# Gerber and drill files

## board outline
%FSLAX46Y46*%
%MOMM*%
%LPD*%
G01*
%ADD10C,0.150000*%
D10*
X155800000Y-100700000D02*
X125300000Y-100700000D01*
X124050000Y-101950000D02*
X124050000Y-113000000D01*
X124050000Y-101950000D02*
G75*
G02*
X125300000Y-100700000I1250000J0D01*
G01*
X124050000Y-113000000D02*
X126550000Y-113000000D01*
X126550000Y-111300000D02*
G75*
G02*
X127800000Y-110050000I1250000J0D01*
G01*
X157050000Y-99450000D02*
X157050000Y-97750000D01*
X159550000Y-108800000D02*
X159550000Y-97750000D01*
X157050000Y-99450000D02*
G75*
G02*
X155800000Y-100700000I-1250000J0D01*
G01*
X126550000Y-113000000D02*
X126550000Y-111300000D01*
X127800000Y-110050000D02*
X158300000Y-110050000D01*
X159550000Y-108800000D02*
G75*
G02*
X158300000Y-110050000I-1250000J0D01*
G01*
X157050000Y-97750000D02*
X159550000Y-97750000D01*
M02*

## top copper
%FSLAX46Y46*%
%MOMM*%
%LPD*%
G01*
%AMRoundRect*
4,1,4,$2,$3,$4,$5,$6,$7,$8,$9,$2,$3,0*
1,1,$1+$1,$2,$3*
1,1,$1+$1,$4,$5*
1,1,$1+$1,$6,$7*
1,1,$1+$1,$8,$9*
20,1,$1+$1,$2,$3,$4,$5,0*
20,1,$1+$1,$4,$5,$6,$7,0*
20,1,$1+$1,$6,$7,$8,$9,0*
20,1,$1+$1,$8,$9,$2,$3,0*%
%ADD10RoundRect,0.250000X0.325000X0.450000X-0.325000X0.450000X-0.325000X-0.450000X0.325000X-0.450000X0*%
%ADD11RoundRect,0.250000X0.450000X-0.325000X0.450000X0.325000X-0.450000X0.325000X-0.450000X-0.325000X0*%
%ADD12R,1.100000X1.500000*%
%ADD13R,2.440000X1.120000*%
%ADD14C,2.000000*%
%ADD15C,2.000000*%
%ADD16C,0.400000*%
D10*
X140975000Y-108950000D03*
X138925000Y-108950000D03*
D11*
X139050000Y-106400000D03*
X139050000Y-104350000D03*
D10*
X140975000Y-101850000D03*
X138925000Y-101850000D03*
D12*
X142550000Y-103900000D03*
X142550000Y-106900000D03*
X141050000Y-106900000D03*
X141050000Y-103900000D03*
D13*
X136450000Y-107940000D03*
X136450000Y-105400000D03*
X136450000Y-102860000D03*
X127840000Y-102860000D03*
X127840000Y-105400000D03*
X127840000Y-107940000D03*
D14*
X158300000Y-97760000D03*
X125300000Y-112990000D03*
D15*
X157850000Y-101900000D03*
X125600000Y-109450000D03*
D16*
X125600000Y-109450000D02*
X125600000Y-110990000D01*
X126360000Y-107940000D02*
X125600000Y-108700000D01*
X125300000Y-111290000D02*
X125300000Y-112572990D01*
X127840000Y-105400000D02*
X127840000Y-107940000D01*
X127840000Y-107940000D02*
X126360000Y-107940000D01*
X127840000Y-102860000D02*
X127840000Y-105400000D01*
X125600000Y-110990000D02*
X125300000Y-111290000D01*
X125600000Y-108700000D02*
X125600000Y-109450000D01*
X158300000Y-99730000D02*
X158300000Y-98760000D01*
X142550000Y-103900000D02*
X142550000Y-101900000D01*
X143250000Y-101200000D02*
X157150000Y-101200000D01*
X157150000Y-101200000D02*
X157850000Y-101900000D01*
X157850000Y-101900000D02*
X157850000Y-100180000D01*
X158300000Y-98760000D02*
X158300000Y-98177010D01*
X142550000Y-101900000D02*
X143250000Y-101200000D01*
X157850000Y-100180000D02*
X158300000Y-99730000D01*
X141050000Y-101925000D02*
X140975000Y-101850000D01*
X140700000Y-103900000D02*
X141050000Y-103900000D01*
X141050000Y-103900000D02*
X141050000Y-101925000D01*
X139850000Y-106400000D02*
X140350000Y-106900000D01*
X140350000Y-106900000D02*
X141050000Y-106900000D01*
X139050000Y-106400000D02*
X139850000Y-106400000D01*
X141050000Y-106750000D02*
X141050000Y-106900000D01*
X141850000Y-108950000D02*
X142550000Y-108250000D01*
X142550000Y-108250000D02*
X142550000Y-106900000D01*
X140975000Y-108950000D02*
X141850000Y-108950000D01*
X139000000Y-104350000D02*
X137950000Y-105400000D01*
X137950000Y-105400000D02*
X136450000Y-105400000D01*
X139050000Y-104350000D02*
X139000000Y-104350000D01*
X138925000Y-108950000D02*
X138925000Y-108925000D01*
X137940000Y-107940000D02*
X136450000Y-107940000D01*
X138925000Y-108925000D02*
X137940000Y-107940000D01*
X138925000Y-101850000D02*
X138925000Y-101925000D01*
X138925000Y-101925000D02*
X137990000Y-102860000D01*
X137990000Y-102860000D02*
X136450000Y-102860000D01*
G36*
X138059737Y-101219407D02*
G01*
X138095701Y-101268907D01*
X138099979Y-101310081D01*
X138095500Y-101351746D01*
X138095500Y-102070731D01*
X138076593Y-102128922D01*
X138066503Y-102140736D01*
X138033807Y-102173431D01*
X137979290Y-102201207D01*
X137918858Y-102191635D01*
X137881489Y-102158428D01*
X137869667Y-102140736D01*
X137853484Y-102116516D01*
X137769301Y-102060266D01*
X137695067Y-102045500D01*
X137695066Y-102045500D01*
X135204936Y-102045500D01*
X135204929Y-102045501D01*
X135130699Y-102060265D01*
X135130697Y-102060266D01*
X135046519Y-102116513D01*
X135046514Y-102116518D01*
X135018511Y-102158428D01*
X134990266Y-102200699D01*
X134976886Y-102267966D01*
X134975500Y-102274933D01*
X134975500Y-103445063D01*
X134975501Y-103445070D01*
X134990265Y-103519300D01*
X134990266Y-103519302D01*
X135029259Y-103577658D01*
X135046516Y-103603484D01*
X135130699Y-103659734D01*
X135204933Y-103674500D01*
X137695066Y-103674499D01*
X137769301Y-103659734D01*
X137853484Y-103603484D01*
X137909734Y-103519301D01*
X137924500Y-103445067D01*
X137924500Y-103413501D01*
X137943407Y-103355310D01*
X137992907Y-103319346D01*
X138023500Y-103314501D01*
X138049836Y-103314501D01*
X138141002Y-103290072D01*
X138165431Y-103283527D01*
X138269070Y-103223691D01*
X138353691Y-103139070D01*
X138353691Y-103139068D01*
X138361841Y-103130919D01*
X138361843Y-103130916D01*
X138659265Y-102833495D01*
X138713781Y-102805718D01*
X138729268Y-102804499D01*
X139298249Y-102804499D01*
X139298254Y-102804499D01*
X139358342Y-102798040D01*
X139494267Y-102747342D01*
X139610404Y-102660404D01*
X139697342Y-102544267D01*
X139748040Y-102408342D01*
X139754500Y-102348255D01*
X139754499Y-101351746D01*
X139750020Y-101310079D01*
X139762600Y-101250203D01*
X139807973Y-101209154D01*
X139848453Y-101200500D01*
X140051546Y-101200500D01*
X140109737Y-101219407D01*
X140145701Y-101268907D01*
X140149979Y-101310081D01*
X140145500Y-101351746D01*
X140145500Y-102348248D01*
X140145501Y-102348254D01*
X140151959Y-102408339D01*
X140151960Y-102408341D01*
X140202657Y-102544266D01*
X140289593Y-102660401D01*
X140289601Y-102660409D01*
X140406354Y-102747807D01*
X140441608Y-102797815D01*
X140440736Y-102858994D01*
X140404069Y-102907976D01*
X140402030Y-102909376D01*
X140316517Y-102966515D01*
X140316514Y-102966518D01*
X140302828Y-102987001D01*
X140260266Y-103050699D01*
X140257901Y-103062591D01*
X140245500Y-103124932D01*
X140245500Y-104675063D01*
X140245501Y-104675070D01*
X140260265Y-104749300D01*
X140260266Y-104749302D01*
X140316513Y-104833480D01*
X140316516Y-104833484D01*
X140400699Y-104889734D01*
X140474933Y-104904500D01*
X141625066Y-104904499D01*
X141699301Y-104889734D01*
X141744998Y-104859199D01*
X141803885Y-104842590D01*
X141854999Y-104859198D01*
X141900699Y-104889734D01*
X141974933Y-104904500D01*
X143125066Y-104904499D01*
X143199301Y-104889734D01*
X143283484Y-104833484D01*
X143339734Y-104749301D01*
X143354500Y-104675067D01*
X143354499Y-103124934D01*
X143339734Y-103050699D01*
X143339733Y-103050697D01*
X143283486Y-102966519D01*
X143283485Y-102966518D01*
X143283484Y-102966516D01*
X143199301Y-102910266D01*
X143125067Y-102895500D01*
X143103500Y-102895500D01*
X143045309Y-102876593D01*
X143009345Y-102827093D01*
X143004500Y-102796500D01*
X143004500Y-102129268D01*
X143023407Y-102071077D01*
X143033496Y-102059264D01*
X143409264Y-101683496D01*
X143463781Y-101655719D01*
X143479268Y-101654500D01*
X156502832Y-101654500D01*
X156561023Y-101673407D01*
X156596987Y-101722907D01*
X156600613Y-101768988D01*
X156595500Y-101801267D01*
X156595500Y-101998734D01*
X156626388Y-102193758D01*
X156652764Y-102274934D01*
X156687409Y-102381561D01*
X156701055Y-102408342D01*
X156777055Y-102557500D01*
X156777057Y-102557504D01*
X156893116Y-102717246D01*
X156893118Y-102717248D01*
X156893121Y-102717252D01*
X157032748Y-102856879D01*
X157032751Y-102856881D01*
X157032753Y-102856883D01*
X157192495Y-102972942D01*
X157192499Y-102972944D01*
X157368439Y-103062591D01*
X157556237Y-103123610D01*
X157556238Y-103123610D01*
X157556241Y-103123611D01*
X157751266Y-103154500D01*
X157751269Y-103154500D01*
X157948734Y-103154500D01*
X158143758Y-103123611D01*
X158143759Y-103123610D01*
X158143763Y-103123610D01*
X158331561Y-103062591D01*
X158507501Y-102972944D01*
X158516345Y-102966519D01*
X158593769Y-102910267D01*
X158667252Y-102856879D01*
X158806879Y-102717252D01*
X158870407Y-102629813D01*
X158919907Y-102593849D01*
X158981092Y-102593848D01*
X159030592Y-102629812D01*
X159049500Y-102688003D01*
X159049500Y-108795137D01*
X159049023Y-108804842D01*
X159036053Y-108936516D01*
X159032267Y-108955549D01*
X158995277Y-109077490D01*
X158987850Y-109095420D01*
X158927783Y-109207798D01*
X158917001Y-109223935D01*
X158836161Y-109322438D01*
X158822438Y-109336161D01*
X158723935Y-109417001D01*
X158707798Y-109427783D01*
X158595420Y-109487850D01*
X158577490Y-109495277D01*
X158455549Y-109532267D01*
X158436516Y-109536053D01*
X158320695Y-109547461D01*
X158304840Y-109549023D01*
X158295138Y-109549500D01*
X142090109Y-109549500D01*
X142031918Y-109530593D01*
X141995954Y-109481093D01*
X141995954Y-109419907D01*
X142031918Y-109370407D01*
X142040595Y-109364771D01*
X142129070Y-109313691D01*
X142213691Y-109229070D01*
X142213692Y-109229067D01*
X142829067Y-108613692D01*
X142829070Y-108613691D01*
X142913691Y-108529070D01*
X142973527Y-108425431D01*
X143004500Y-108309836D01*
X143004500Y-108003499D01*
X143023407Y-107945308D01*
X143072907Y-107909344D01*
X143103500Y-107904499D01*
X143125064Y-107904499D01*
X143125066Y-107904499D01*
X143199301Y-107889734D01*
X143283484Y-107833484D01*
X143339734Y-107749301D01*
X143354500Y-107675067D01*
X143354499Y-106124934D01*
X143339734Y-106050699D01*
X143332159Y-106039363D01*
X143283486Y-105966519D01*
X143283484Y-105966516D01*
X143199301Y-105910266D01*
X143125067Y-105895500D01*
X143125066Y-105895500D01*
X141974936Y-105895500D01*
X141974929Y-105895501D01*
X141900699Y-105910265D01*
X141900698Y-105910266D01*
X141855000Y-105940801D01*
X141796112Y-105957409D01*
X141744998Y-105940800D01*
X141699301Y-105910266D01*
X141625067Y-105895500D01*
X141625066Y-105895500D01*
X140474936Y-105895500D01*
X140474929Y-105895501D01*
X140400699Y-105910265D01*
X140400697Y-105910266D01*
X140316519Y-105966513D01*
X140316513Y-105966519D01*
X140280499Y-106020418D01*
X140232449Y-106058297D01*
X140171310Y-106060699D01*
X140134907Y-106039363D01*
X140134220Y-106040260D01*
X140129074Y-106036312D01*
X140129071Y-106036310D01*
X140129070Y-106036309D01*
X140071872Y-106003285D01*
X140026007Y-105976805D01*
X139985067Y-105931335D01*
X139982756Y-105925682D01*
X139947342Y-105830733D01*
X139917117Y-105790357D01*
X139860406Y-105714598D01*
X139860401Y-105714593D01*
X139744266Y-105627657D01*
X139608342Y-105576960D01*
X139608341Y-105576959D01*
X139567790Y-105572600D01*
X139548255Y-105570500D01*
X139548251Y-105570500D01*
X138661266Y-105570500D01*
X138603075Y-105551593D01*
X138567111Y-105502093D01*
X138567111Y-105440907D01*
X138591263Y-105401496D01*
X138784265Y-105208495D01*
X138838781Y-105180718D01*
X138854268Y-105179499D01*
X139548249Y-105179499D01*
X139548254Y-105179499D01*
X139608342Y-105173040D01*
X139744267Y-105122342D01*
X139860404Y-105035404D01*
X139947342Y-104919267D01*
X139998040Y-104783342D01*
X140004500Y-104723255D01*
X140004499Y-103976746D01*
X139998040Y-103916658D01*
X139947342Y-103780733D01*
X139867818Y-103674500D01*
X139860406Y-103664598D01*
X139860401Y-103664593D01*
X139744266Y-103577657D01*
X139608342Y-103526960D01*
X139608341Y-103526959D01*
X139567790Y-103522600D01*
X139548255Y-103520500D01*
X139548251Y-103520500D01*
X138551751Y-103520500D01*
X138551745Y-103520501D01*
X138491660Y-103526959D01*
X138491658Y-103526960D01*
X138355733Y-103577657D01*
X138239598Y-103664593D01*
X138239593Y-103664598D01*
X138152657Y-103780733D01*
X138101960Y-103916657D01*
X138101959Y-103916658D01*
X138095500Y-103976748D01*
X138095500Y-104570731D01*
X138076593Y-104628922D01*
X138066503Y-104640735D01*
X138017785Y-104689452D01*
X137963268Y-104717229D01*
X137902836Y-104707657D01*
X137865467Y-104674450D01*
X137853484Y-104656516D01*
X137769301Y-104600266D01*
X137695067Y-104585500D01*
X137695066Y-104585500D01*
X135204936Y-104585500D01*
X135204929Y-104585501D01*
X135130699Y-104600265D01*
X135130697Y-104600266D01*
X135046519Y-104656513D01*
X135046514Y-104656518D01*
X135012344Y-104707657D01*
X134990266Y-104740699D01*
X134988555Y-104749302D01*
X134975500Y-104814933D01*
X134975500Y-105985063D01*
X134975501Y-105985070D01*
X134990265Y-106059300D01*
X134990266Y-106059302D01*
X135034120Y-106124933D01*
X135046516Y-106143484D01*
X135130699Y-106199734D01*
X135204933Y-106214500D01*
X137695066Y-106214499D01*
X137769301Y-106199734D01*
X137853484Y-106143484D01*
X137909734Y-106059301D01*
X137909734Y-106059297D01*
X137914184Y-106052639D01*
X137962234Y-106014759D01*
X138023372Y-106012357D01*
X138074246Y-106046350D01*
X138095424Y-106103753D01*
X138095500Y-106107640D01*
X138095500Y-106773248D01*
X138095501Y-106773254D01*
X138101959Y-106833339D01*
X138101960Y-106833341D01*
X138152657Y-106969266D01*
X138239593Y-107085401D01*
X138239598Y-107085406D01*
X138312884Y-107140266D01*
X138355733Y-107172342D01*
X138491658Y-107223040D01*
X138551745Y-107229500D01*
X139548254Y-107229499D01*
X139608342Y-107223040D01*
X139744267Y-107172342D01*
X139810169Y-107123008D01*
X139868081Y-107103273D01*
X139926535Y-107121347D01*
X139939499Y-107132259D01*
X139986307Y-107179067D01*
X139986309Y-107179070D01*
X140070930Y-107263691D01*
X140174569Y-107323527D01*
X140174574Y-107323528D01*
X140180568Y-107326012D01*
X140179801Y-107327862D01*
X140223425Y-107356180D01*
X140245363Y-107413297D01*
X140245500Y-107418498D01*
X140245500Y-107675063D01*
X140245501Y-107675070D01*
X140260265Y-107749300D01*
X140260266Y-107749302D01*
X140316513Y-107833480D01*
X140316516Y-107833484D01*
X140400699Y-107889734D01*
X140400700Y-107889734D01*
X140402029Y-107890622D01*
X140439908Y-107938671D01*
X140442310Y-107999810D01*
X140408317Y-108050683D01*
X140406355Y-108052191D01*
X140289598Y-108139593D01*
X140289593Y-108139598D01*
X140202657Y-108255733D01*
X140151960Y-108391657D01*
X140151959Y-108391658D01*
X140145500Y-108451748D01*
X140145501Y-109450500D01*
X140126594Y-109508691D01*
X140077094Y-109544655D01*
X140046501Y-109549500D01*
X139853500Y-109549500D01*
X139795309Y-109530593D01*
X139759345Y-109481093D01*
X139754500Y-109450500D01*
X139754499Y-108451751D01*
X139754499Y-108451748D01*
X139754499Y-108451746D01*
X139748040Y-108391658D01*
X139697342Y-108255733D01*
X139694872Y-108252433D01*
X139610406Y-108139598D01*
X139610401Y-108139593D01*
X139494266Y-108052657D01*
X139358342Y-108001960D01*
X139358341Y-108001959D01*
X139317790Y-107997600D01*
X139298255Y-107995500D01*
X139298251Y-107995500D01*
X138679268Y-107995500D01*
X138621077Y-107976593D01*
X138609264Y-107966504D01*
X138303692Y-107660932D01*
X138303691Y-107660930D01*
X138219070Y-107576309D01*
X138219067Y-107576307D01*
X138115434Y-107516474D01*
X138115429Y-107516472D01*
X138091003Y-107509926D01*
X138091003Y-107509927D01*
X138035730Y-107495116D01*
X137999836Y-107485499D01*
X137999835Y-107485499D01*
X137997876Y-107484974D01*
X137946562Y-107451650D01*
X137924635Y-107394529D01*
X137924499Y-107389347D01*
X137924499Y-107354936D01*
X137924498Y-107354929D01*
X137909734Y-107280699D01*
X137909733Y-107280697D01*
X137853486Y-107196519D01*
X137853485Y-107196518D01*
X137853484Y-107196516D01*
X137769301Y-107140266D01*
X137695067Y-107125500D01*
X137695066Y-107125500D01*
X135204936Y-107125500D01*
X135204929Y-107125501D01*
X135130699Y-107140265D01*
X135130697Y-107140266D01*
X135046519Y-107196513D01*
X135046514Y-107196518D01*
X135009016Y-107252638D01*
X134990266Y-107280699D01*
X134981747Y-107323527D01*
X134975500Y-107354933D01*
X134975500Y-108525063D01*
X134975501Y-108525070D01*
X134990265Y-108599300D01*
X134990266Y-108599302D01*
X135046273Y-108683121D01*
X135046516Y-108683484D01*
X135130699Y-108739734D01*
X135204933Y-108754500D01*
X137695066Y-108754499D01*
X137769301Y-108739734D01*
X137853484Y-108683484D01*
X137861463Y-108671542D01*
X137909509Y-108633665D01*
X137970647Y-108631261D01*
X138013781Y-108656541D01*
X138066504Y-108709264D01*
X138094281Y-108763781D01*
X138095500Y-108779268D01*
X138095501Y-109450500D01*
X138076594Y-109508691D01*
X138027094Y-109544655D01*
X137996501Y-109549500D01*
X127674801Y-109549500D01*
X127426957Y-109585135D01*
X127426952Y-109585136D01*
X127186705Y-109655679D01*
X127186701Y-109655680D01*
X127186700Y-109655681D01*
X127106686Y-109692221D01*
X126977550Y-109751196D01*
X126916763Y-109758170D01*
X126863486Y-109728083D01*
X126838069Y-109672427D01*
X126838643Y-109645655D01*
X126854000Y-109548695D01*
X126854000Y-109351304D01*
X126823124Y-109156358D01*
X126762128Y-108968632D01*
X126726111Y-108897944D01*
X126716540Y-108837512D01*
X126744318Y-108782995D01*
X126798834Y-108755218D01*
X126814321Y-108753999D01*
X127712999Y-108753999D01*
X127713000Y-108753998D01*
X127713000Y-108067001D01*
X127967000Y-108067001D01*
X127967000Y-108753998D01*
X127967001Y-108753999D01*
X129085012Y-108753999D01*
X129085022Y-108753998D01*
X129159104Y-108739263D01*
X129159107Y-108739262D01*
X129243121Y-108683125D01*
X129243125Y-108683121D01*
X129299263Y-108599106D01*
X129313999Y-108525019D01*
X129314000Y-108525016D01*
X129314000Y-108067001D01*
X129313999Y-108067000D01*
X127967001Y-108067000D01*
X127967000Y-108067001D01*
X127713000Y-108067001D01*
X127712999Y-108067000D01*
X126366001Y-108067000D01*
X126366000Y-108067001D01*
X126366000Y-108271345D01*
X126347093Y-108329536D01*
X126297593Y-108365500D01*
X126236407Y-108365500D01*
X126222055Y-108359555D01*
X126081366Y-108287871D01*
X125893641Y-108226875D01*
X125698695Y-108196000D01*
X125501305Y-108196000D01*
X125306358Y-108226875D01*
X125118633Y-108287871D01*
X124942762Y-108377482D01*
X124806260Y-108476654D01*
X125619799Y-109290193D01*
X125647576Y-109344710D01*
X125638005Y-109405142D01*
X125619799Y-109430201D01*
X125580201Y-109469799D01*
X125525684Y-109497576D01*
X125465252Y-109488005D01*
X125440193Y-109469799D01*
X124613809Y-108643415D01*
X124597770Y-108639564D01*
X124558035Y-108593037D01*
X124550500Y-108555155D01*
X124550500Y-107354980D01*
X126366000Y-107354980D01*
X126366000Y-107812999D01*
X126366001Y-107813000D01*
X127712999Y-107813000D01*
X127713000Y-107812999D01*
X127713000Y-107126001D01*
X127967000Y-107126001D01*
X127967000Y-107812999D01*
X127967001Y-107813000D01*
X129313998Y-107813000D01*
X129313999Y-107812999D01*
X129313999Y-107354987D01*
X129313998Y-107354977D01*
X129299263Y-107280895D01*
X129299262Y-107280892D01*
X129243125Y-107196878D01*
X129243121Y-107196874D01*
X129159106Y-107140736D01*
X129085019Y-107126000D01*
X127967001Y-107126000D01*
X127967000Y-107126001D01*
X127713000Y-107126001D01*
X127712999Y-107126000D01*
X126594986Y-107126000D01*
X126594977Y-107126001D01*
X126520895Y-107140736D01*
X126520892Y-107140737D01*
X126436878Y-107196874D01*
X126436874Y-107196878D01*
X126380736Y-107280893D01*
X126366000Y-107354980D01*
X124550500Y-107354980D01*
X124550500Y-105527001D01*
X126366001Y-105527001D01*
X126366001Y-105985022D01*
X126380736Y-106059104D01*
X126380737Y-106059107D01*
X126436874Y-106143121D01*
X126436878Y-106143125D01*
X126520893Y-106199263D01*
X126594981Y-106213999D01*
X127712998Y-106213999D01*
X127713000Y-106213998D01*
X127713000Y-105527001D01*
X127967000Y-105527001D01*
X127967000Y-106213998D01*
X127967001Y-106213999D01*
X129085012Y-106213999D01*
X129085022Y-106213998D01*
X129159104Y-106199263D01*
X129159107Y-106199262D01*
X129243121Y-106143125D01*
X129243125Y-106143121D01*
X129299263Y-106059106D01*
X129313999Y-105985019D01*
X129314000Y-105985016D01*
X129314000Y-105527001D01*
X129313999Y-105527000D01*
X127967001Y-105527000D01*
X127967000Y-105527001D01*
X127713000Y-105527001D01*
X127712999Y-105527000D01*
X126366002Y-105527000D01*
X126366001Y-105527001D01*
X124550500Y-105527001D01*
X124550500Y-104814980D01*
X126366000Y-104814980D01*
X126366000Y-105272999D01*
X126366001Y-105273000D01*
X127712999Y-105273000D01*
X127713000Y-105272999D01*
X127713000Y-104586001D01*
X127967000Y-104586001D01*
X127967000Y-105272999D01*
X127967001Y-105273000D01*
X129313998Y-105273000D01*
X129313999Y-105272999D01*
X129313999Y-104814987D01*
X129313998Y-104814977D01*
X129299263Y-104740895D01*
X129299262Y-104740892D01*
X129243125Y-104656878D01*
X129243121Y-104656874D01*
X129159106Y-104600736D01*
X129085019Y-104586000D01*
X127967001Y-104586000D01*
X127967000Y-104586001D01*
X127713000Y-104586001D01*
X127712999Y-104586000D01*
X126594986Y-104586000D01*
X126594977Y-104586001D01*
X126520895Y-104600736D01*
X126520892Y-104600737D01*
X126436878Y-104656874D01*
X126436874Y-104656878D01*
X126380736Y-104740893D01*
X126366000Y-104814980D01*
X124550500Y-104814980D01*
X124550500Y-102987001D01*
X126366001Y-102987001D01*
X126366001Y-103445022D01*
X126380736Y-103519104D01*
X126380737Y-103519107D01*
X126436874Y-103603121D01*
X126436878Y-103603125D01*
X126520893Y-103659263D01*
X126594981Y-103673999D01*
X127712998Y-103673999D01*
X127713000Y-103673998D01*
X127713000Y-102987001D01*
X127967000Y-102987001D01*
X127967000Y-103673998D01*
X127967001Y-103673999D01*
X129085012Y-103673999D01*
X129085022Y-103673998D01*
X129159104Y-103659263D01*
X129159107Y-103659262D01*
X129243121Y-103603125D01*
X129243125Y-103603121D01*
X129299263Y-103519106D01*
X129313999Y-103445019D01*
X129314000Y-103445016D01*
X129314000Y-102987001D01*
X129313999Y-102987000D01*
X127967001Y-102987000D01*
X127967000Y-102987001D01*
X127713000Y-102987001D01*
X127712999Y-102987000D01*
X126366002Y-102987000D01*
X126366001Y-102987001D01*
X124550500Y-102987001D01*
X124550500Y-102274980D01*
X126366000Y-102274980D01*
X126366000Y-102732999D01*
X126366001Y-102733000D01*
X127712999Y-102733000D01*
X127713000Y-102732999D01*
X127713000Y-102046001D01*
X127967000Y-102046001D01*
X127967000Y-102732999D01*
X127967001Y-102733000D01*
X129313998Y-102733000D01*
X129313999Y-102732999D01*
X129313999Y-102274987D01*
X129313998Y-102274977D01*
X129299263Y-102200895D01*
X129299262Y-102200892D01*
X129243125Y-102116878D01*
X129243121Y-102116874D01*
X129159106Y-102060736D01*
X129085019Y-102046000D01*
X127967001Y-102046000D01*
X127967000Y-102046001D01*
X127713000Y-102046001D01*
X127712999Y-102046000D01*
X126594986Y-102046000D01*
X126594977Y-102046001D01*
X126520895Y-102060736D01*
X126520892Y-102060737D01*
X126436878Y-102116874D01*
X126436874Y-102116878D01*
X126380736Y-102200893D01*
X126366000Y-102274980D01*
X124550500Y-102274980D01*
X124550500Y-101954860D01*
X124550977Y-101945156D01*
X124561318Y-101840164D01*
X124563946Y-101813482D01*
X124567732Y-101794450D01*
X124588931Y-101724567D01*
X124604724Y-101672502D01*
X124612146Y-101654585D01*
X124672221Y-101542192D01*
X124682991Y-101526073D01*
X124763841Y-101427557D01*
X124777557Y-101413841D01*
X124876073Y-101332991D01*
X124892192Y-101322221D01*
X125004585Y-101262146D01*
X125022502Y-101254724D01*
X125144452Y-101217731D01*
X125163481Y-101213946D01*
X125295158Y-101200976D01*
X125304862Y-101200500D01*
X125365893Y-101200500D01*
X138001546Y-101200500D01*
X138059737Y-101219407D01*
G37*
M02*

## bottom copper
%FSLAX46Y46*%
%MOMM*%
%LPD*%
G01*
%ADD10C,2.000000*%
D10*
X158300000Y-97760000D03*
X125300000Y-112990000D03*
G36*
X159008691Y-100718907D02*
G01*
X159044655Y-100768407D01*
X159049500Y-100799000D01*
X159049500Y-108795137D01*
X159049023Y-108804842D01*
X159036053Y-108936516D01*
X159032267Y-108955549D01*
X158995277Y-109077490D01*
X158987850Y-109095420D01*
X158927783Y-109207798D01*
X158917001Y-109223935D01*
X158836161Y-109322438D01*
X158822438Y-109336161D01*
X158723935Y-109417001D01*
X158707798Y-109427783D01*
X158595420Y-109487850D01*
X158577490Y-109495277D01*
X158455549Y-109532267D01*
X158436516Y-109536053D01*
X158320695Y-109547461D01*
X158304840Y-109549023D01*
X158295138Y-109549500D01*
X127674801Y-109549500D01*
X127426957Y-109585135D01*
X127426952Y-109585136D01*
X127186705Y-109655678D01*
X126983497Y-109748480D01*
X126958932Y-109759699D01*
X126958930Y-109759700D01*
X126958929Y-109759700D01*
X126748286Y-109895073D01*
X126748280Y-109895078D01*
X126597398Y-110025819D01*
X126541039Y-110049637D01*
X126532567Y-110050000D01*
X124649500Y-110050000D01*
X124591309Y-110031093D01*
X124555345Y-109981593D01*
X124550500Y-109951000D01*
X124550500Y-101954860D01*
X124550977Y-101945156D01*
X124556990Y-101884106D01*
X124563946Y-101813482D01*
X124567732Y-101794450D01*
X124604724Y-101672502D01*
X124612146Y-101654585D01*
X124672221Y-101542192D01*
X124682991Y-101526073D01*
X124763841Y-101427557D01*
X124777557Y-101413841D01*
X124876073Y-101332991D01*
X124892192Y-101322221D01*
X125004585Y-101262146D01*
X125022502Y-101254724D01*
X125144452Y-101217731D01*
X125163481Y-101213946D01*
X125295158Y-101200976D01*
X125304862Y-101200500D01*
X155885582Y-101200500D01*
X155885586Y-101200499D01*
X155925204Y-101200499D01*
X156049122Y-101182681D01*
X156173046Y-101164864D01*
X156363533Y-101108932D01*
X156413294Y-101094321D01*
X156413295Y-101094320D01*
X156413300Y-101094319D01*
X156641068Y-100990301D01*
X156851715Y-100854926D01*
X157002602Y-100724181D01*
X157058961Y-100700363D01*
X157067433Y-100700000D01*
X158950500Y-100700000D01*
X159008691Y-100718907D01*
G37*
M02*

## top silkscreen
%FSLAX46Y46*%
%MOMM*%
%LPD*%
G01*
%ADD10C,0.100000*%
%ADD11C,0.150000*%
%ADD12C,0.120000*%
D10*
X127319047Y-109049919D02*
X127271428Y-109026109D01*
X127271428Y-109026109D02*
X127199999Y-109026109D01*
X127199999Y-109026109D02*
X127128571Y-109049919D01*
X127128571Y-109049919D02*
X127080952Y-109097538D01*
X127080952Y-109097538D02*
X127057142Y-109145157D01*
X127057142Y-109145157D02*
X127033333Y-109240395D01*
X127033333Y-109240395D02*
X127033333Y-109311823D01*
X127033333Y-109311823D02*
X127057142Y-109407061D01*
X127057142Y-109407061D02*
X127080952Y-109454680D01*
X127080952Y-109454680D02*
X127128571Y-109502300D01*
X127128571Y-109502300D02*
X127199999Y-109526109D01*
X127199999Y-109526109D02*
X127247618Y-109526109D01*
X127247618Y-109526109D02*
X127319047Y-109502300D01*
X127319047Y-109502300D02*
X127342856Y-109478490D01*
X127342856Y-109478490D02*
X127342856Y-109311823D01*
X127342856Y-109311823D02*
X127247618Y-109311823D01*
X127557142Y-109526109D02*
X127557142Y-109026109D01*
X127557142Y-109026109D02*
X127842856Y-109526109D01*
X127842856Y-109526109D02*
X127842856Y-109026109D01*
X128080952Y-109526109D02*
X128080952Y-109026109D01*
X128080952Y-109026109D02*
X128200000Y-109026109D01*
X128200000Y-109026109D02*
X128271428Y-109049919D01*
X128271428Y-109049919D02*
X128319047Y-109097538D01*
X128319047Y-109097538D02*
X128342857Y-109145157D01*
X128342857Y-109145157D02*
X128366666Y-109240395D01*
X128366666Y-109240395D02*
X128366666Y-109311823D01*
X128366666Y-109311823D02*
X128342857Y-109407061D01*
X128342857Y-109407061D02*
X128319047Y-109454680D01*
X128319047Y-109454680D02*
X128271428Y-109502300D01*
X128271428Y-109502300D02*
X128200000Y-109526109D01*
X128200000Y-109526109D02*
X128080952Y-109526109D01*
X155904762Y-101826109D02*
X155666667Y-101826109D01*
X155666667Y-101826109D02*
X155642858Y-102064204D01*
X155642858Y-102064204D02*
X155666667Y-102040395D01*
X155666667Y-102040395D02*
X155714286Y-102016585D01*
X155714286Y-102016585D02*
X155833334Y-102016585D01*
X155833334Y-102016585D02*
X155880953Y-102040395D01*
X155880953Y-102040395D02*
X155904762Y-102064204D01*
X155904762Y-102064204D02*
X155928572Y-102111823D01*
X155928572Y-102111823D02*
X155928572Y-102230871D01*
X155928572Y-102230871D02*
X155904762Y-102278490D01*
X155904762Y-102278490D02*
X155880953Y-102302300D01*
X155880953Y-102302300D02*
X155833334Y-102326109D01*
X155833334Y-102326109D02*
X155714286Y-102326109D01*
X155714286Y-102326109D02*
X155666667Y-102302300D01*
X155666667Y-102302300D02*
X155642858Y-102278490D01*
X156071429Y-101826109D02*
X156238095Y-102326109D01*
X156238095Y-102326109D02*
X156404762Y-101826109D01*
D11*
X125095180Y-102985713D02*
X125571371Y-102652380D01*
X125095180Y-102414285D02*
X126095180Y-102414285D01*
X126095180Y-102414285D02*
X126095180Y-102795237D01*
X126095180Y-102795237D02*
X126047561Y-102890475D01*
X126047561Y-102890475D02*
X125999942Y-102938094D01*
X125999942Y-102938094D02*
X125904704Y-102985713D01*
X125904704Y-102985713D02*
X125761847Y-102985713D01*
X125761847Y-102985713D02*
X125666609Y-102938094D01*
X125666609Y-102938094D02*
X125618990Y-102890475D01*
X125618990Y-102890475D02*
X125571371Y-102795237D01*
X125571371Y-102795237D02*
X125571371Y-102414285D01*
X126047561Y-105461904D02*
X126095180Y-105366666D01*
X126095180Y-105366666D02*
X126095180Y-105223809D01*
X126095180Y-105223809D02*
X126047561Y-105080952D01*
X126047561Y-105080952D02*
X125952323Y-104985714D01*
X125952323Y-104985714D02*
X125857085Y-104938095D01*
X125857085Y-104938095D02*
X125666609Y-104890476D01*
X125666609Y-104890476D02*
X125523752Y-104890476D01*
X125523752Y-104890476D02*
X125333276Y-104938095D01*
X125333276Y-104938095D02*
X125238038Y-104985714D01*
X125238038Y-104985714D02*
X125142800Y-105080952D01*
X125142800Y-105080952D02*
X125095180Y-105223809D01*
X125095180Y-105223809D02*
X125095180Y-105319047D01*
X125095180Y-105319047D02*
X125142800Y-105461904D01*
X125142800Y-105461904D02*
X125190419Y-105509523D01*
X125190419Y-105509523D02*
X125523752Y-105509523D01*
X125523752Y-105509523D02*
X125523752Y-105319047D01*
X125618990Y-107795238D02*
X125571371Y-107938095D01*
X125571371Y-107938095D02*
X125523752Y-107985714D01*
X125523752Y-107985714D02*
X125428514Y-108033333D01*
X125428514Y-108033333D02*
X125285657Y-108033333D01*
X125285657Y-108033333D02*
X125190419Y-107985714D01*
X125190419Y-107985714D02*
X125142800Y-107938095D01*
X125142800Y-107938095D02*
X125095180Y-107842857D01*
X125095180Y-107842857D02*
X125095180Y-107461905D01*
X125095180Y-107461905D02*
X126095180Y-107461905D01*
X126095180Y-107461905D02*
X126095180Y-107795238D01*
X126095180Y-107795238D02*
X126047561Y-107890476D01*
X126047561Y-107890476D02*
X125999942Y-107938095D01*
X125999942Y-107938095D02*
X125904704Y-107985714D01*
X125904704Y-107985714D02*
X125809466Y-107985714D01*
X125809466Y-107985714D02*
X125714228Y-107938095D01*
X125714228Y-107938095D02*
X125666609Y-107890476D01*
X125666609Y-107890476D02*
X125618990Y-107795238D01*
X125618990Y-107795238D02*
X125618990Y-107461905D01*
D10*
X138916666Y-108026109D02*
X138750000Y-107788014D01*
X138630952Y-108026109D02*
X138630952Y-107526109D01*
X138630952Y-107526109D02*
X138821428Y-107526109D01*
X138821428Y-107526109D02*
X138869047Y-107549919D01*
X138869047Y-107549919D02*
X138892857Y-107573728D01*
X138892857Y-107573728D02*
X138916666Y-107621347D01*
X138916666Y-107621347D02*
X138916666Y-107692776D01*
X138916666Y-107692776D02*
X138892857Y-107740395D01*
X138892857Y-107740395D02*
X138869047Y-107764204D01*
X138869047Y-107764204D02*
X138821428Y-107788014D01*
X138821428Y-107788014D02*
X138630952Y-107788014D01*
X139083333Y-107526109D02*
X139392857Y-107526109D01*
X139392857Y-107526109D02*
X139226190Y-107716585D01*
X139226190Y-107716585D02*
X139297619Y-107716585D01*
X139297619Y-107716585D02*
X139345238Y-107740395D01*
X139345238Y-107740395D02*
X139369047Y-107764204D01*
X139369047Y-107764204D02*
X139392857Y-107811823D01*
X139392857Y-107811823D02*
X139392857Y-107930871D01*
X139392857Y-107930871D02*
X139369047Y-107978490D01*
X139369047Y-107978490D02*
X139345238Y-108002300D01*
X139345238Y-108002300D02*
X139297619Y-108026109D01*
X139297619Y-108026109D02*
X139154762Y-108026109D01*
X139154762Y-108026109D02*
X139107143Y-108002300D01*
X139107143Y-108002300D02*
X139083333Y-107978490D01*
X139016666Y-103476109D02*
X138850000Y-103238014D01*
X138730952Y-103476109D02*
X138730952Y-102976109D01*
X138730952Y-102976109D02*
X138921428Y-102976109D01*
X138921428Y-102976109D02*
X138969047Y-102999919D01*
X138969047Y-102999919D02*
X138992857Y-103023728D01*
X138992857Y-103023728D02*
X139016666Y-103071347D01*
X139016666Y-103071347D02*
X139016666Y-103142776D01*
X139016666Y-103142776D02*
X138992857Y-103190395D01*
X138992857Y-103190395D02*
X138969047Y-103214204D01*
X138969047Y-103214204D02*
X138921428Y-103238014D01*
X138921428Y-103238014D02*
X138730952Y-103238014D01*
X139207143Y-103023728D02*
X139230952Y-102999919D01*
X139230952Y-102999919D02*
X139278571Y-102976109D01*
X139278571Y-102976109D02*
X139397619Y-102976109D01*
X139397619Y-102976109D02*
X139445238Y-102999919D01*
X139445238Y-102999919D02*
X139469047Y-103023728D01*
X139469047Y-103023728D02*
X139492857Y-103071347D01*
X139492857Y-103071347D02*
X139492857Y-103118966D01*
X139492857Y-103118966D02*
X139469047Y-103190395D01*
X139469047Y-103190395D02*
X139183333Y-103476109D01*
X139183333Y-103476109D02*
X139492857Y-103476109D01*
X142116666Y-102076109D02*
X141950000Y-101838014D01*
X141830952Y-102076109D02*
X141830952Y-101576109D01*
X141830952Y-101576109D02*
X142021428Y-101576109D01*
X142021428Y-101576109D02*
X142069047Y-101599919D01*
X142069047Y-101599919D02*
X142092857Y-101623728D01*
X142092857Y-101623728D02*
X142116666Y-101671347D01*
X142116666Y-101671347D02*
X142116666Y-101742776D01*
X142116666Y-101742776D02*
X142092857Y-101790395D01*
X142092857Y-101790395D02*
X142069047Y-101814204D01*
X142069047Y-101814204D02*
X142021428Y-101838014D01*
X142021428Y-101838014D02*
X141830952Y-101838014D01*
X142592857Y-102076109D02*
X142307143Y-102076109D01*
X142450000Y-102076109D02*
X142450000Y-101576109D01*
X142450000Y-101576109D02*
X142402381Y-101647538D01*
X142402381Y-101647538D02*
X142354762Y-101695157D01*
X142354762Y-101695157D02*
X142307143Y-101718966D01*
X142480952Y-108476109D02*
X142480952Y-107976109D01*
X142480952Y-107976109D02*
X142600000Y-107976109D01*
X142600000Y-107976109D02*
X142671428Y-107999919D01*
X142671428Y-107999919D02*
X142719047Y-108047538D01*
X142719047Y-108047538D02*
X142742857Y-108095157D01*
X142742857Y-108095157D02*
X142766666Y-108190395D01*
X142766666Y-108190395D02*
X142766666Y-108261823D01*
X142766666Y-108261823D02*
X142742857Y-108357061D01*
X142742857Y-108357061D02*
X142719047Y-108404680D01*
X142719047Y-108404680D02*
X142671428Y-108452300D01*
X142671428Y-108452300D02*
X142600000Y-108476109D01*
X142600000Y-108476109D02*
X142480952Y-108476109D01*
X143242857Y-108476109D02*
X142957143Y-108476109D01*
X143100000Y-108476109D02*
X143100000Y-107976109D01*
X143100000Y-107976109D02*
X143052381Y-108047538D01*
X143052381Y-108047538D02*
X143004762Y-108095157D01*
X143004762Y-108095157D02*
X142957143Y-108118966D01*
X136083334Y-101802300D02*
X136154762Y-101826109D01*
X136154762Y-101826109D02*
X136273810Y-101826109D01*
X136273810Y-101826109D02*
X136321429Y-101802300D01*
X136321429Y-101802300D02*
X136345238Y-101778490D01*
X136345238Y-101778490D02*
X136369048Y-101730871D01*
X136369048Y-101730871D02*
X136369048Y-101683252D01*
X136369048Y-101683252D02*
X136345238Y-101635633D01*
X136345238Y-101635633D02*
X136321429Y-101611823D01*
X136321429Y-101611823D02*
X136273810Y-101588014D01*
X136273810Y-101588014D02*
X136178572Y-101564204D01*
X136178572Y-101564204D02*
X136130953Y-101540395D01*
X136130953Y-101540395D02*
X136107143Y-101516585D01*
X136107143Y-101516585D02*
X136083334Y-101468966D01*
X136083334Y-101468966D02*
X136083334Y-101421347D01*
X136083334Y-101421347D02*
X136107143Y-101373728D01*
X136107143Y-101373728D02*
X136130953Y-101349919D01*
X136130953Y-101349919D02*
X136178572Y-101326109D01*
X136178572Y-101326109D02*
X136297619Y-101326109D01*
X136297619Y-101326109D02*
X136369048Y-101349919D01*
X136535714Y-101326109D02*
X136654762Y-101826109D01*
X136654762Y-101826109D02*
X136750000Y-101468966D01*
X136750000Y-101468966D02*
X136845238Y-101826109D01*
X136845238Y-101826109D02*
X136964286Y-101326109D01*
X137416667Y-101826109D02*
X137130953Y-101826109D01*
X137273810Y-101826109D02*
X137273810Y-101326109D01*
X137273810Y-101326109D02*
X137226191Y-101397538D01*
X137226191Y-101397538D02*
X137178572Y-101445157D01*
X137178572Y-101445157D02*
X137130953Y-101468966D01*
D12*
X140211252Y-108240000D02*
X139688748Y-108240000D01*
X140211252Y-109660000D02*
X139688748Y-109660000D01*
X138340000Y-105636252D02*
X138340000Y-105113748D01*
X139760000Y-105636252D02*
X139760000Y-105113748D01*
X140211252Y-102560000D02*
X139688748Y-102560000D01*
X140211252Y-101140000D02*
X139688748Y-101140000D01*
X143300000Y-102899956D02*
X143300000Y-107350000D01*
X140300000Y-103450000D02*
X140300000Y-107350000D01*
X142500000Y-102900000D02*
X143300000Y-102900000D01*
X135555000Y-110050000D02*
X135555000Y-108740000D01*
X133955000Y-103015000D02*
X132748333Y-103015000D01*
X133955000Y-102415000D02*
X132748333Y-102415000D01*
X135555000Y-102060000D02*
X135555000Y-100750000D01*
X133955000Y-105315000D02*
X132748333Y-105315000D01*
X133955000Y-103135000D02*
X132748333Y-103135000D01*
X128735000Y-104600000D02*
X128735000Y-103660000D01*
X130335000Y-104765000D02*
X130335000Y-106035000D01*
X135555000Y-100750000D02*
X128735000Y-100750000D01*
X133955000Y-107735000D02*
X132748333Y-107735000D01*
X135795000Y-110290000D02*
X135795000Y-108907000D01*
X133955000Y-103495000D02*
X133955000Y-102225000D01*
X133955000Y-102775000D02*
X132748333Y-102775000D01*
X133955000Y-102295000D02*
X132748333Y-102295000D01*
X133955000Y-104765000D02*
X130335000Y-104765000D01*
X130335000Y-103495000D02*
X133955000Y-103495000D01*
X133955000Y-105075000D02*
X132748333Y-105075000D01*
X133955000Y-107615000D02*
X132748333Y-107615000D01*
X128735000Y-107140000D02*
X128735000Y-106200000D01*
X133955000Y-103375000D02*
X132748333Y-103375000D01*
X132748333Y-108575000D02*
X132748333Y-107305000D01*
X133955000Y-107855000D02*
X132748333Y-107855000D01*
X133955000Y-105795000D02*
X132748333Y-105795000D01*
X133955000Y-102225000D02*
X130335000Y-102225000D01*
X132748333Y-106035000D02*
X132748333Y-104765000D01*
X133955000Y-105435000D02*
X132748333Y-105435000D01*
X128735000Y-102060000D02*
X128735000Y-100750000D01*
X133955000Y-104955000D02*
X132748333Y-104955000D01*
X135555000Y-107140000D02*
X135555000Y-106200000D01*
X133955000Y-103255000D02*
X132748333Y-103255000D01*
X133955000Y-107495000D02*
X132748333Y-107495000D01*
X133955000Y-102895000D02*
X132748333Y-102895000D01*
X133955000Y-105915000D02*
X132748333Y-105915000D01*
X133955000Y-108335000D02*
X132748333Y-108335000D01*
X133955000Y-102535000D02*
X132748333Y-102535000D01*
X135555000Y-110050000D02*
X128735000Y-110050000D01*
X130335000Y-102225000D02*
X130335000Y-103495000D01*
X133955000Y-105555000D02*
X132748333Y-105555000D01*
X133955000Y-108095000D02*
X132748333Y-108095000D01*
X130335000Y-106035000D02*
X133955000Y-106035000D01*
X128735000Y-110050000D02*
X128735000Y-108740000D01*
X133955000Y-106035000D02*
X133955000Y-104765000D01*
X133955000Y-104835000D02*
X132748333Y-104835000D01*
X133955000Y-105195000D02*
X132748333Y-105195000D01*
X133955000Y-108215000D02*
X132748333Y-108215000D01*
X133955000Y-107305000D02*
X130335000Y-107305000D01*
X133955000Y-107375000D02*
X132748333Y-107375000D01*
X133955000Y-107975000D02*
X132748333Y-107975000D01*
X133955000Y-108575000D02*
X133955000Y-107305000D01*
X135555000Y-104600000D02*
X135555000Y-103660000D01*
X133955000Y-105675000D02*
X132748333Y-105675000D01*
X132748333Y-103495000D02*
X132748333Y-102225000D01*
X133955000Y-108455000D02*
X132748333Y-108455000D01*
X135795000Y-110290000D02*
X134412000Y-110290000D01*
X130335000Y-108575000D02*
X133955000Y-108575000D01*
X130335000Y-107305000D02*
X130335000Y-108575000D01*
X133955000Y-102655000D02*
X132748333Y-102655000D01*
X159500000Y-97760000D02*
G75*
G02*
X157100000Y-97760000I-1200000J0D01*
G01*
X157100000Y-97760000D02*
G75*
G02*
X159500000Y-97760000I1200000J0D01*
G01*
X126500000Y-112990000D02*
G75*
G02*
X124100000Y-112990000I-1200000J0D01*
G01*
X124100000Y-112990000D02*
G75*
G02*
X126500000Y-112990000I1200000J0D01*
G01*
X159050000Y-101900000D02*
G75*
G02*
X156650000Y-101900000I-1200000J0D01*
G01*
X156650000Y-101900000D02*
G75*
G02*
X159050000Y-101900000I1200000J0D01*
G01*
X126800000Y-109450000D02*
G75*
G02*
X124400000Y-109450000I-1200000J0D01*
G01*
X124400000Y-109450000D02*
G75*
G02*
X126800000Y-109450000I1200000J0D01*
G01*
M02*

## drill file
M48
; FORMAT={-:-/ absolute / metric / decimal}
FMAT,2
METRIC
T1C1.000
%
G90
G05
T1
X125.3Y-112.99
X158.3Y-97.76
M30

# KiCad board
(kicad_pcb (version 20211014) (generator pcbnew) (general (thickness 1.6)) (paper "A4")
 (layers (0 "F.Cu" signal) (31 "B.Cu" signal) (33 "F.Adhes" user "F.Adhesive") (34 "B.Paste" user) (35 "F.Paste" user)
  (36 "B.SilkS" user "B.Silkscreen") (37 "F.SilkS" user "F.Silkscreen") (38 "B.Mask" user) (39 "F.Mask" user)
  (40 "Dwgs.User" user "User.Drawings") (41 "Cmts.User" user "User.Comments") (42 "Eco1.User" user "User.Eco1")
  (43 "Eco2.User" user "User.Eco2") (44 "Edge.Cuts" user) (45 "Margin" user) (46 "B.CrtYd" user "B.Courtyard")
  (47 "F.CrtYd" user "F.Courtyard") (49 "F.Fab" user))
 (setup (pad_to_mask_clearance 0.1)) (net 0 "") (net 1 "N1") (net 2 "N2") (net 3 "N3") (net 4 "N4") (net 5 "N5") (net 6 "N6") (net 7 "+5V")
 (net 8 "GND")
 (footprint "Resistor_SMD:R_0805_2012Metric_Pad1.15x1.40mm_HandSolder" (layer "F.Cu") (at 139.95 108.95 180)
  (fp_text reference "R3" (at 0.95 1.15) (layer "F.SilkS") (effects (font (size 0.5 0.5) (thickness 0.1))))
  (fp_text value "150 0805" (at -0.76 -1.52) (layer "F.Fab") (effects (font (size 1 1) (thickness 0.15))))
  (fp_line (start -0.261252 0.71) (end 0.261252 0.71) (layer "F.SilkS") (width 0.12))
  (fp_line (start -0.261252 -0.71) (end 0.261252 -0.71) (layer "F.SilkS") (width 0.12))
  (pad "1" smd roundrect locked (at -1.025 0 180) (size 1.15 1.4) (layers "F.Cu" "F.Paste" "F.Mask") (roundrect_rratio 0.217391)
   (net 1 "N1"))
  (pad "2" smd roundrect locked (at 1.025 0 180) (size 1.15 1.4) (layers "F.Cu" "F.Paste" "F.Mask") (roundrect_rratio 0.217391) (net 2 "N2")))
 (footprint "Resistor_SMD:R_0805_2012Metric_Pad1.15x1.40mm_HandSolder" (layer "F.Cu") (at 139.05 105.375 90)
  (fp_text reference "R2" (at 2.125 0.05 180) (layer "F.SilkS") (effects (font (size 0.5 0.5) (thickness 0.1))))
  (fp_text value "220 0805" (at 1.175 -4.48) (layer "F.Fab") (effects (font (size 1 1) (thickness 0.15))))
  (fp_line (start -0.261252 -0.71) (end 0.261252 -0.71) (layer "F.SilkS") (width 0.12))
  (fp_line (start -0.261252 0.71) (end 0.261252 0.71) (layer "F.SilkS") (width 0.12))
  (pad "1" smd roundrect locked (at -1.025 0 90) (size 1.15 1.4) (layers "F.Cu" "F.Paste" "F.Mask") (roundrect_rratio 0.217391) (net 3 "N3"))
  (pad "2" smd roundrect locked (at 1.025 0 90) (size 1.15 1.4) (layers "F.Cu" "F.Paste" "F.Mask") (roundrect_rratio 0.217391) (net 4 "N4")))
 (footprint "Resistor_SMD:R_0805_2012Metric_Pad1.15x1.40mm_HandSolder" (layer "F.Cu") (at 139.95 101.85 180)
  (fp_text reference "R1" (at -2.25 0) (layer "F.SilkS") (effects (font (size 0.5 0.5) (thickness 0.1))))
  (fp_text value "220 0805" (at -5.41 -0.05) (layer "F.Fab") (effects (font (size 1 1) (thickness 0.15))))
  (fp_line (start -0.261252 -0.71) (end 0.261252 -0.71) (layer "F.SilkS") (width 0.12))
  (fp_line (start -0.261252 0.71) (end 0.261252 0.71) (layer "F.SilkS") (width 0.12))
  (pad "1" smd roundrect locked (at -1.025 0 180) (size 1.15 1.4) (layers "F.Cu" "F.Paste" "F.Mask") (roundrect_rratio 0.217391)
   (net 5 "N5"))
  (pad "2" smd roundrect locked (at 1.025 0 180) (size 1.15 1.4) (layers "F.Cu" "F.Paste" "F.Mask") (roundrect_rratio 0.217391) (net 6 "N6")))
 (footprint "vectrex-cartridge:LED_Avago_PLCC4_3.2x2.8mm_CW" (layer "F.Cu") (at 141.8 105.4 -90)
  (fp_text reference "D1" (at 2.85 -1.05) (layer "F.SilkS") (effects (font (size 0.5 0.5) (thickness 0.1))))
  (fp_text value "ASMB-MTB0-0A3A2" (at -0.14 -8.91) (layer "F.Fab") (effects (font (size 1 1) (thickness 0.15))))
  (fp_line (start -2.500044 -1.5) (end 1.95 -1.5) (layer "F.SilkS") (width 0.12))
  (fp_line (start -1.95 1.5) (end 1.95 1.5) (layer "F.SilkS") (width 0.12))
  (fp_line (start -2.5 -0.7) (end -2.5 -1.5) (layer "F.SilkS") (width 0.12))
  (pad "1" smd rect locked (at -1.5 -0.75 270) (size 1.5 1.1) (layers "F.Cu" "F.Paste" "F.Mask") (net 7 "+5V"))
  (pad "2" smd rect locked (at 1.5 -0.75 270) (size 1.5 1.1) (layers "F.Cu" "F.Paste" "F.Mask") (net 1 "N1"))
  (pad "3" smd rect locked (at 1.5 0.75 270) (size 1.5 1.1) (layers "F.Cu" "F.Paste" "F.Mask") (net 3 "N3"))
  (pad "4" smd rect locked (at -1.5 0.75 270) (size 1.5 1.1) (layers "F.Cu" "F.Paste" "F.Mask") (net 5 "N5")))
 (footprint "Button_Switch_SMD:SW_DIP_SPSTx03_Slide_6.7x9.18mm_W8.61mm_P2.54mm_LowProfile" (layer "F.Cu") (at 132.145 105.4 180)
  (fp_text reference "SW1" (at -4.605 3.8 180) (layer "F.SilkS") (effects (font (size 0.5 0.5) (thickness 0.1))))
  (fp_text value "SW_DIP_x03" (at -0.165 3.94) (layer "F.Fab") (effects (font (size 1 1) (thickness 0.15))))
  (fp_line (start -3.41 -4.65) (end -3.41 -3.34) (layer "F.SilkS") (width 0.12))
  (fp_line (start -1.81 2.385) (end -0.603333 2.385) (layer "F.SilkS") (width 0.12))
  (fp_line (start -1.81 2.985) (end -0.603333 2.985) (layer "F.SilkS") (width 0.12))
  (fp_line (start -3.41 3.34) (end -3.41 4.65) (layer "F.SilkS") (width 0.12))
  (fp_line (start -1.81 0.085) (end -0.603333 0.085) (layer "F.SilkS") (width 0.12))
  (fp_line (start -1.81 2.265) (end -0.603333 2.265) (layer "F.SilkS") (width 0.12))
  (fp_line (start 3.41 0.8) (end 3.41 1.74) (layer "F.SilkS") (width 0.12))
  (fp_line (start 1.81 0.635) (end 1.81 -0.635) (layer "F.SilkS") (width 0.12))
  (fp_line (start -3.41 4.65) (end 3.41 4.65) (layer "F.SilkS") (width 0.12))
  (fp_line (start -1.81 -2.335) (end -0.603333 -2.335) (layer "F.SilkS") (width 0.12))
  (fp_line (start -3.65 -4.89) (end -3.65 -3.507) (layer "F.SilkS") (width 0.12))
  (fp_line (start -1.81 1.905) (end -1.81 3.175) (layer "F.SilkS") (width 0.12))
  (fp_line (start -1.81 2.625) (end -0.603333 2.625) (layer "F.SilkS") (width 0.12))
  (fp_line (start -1.81 3.105) (end -0.603333 3.105) (layer "F.SilkS") (width 0.12))
  (fp_line (start -1.81 0.635) (end 1.81 0.635) (layer "F.SilkS") (width 0.12))
  (fp_line (start 1.81 1.905) (end -1.81 1.905) (layer "F.SilkS") (width 0.12))
  (fp_line (start -1.81 0.325) (end -0.603333 0.325) (layer "F.SilkS") (width 0.12))
  (fp_line (start -1.81 -2.215) (end -0.603333 -2.215) (layer "F.SilkS") (width 0.12))
  (fp_line (start 3.41 -1.74) (end 3.41 -0.8) (layer "F.SilkS") (width 0.12))
  (fp_line (start -1.81 2.025) (end -0.603333 2.025) (layer "F.SilkS") (width 0.12))
  (fp_line (start -0.603333 -3.175) (end -0.603333 -1.905) (layer "F.SilkS") (width 0.12))
  (fp_line (start -1.81 -2.455) (end -0.603333 -2.455) (layer "F.SilkS") (width 0.12))
  (fp_line (start -1.81 -0.395) (end -0.603333 -0.395) (layer "F.SilkS") (width 0.12))
  (fp_line (start -1.81 3.175) (end 1.81 3.175) (layer "F.SilkS") (width 0.12))
  (fp_line (start -0.603333 -0.635) (end -0.603333 0.635) (layer "F.SilkS") (width 0.12))
  (fp_line (start -1.81 -0.035) (end -0.603333 -0.035) (layer "F.SilkS") (width 0.12))
  (fp_line (start 3.41 3.34) (end 3.41 4.65) (layer "F.SilkS") (width 0.12))
  (fp_line (start -1.81 0.445) (end -0.603333 0.445) (layer "F.SilkS") (width 0.12))
  (fp_line (start -3.41 -1.74) (end -3.41 -0.8) (layer "F.SilkS") (width 0.12))
  (fp_line (start -1.81 2.145) (end -0.603333 2.145) (layer "F.SilkS") (width 0.12))
  (fp_line (start -1.81 -2.095) (end -0.603333 -2.095) (layer "F.SilkS") (width 0.12))
  (fp_line (start -1.81 2.505) (end -0.603333 2.505) (layer "F.SilkS") (width 0.12))
  (fp_line (start -1.81 -0.515) (end -0.603333 -0.515) (layer "F.SilkS") (width 0.12))
  (fp_line (start -1.81 -2.935) (end -0.603333 -2.935) (layer "F.SilkS") (width 0.12))
  (fp_line (start -1.81 2.865) (end -0.603333 2.865) (layer "F.SilkS") (width 0.12))
  (fp_line (start -3.41 -4.65) (end 3.41 -4.65) (layer "F.SilkS") (width 0.12))
  (fp_line (start 1.81 3.175) (end 1.81 1.905) (layer "F.SilkS") (width 0.12))
  (fp_line (start -1.81 -0.155) (end -0.603333 -0.155) (layer "F.SilkS") (width 0.12))
  (fp_line (start -1.81 -2.695) (end -0.603333 -2.695) (layer "F.SilkS") (width 0.12))
  (fp_line (start 1.81 -0.635) (end -1.81 -0.635) (layer "F.SilkS") (width 0.12))
  (fp_line (start 3.41 -4.65) (end 3.41 -3.34) (layer "F.SilkS") (width 0.12))
  (fp_line (start -1.81 -0.635) (end -1.81 0.635) (layer "F.SilkS") (width 0.12))
  (fp_line (start -1.81 0.565) (end -0.603333 0.565) (layer "F.SilkS") (width 0.12))
  (fp_line (start -1.81 0.205) (end -0.603333 0.205) (layer "F.SilkS") (width 0.12))
  (fp_line (start -1.81 -2.815) (end -0.603333 -2.815) (layer "F.SilkS") (width 0.12))
  (fp_line (start -1.81 -1.905) (end 1.81 -1.905) (layer "F.SilkS") (width 0.12))
  (fp_line (start -1.81 -1.975) (end -0.603333 -1.975) (layer "F.SilkS") (width 0.12))
  (fp_line (start -1.81 -2.575) (end -0.603333 -2.575) (layer "F.SilkS") (width 0.12))
  (fp_line (start -1.81 -3.175) (end -1.81 -1.905) (layer "F.SilkS") (width 0.12))
  (fp_line (start -3.41 0.8) (end -3.41 1.74) (layer "F.SilkS") (width 0.12))
  (fp_line (start -1.81 -0.275) (end -0.603333 -0.275) (layer "F.SilkS") (width 0.12))
  (fp_line (start -0.603333 1.905) (end -0.603333 3.175) (layer "F.SilkS") (width 0.12))
  (fp_line (start -1.81 -3.055) (end -0.603333 -3.055) (layer "F.SilkS") (width 0.12))
  (fp_line (start -3.65 -4.89) (end -2.267 -4.89) (layer "F.SilkS") (width 0.12))
  (fp_line (start 1.81 -3.175) (end -1.81 -3.175) (layer "F.SilkS") (width 0.12))
  (fp_line (start 1.81 -1.905) (end 1.81 -3.175) (layer "F.SilkS") (width 0.12))
  (fp_line (start -1.81 2.745) (end -0.603333 2.745) (layer "F.SilkS") (width 0.12))
  (pad "1" smd rect locked (at -4.305 -2.54 180) (size 2.44 1.12) (layers "F.Cu" "F.Paste" "F.Mask") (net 2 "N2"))
  (pad "2" smd rect locked (at -4.305 0 180) (size 2.44 1.12) (layers "F.Cu" "F.Paste" "F.Mask") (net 4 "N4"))
  (pad "3" smd rect locked (at -4.305 2.54 180) (size 2.44 1.12) (layers "F.Cu" "F.Paste" "F.Mask") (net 6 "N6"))
  (pad "4" smd rect locked (at 4.305 2.54 180) (size 2.44 1.12) (layers "F.Cu" "F.Paste" "F.Mask") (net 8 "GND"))
  (pad "5" smd rect locked (at 4.305 0 180) (size 2.44 1.12) (layers "F.Cu" "F.Paste" "F.Mask") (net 8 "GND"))
  (pad "6" smd rect locked (at 4.305 -2.54 180) (size 2.44 1.12) (layers "F.Cu" "F.Paste" "F.Mask") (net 8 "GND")))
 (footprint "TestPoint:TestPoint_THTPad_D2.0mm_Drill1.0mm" (layer "F.Cu") (at 158.3 97.76)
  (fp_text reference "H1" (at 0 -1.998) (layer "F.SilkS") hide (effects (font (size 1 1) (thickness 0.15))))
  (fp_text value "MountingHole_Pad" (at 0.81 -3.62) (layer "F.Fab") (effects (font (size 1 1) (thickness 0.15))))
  (fp_circle (center 0 0) (end 0 1.2) (layer "F.SilkS") (width 0.12) (fill none))
  (pad "1" thru_hole circle locked (at 0 0) (size 2 2) (drill 1) (layers *.Cu *.Mask) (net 7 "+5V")))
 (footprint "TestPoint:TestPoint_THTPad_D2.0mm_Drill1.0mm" (layer "F.Cu") (at 125.3 112.99)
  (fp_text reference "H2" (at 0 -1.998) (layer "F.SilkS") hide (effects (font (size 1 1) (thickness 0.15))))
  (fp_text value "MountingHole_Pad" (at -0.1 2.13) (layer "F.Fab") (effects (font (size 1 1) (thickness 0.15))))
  (fp_circle (center 0 0) (end 0 1.2) (layer "F.SilkS") (width 0.12) (fill none))
  (pad "1" thru_hole circle locked (at 0 0) (size 2 2) (drill 1) (layers *.Cu *.Mask) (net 8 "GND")))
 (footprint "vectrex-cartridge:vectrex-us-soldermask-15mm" (layer "F.Cu") (at 151.1 105.25)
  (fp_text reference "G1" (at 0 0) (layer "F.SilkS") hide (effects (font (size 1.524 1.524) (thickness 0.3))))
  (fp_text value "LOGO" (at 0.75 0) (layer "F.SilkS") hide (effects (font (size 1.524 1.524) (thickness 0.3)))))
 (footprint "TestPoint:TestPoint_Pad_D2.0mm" (layer "F.Cu") (at 157.85 101.9)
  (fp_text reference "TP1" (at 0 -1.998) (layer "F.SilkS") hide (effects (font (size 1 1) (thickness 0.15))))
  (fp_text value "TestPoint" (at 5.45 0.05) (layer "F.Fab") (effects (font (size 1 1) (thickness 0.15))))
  (fp_circle (center 0 0) (end 0 1.2) (layer "F.SilkS") (width 0.12) (fill none))
  (pad "1" smd circle locked (at 0 0) (size 2 2) (layers "F.Cu" "F.Mask") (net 7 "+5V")))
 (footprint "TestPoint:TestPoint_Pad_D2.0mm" (layer "F.Cu") (at 125.6 109.45)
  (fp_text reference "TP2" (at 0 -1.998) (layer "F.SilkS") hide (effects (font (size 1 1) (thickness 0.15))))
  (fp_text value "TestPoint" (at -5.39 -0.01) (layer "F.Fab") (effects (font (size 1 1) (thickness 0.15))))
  (fp_circle (center 0 0) (end 0 1.2) (layer "F.SilkS") (width 0.12) (fill none))
  (pad "1" smd circle locked (at 0 0) (size 2 2) (layers "F.Cu" "F.Mask") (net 8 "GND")))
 (gr_line (start 155.8 100.7) (end 125.3 100.7) (layer "Edge.Cuts") (width 0.15))
 (gr_line (start 124.05 101.95) (end 124.05 113) (layer "Edge.Cuts") (width 0.15))
 (gr_arc (start 124.05 101.95) (mid 124.416117 101.066117) (end 125.3 100.7) (layer "Edge.Cuts") (width 0.15))
 (gr_line (start 124.05 113) (end 126.55 113) (layer "Edge.Cuts") (width 0.15))
 (gr_arc (start 126.55 111.3) (mid 126.916117 110.416117) (end 127.8 110.05) (layer "Edge.Cuts") (width 0.15))
 (gr_line (start 157.05 99.45) (end 157.05 97.75) (layer "Edge.Cuts") (width 0.15))
 (gr_line (start 159.55 108.8) (end 159.55 97.75) (layer "Edge.Cuts") (width 0.15))
 (gr_arc (start 157.05 99.45) (mid 156.683883 100.333883) (end 155.8 100.7) (layer "Edge.Cuts") (width 0.15))
 (gr_line (start 126.55 113) (end 126.55 111.3) (layer "Edge.Cuts") (width 0.15))
 (gr_line (start 127.8 110.05) (end 158.3 110.05) (layer "Edge.Cuts") (width 0.15))
 (gr_arc (start 159.55 108.8) (mid 159.183883 109.683883) (end 158.3 110.05) (layer "Edge.Cuts") (width 0.15))
 (gr_line (start 157.05 97.75) (end 159.55 97.75) (layer "Edge.Cuts") (width 0.15))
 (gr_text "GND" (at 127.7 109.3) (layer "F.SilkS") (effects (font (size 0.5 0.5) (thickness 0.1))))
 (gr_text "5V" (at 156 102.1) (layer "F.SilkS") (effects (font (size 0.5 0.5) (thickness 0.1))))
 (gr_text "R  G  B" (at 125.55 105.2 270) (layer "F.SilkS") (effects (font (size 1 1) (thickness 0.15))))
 (segment (start 125.6 109.45) (end 125.6 110.99) (width 0.4) (layer "F.Cu") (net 8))
 (segment (start 126.36 107.94) (end 125.6 108.7) (width 0.4) (layer "F.Cu") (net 8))
 (segment (start 125.3 111.29) (end 125.3 112.57299) (width 0.4) (layer "F.Cu") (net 8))
 (segment (start 127.84 105.4) (end 127.84 107.94) (width 0.4) (layer "F.Cu") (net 8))
 (segment (start 127.84 107.94) (end 126.36 107.94) (width 0.4) (layer "F.Cu") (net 8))
 (segment (start 127.84 102.86) (end 127.84 105.4) (width 0.4) (layer "F.Cu") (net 8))
 (segment (start 125.6 110.99) (end 125.3 111.29) (width 0.4) (layer "F.Cu") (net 8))
 (segment (start 125.6 108.7) (end 125.6 109.45) (width 0.4) (layer "F.Cu") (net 8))
 (segment (start 158.3 99.73) (end 158.3 98.76) (width 0.4) (layer "F.Cu") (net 7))
 (segment (start 142.55 103.9) (end 142.55 101.9) (width 0.4) (layer "F.Cu") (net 7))
 (segment (start 143.25 101.2) (end 157.15 101.2) (width 0.4) (layer "F.Cu") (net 7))
 (segment (start 157.15 101.2) (end 157.85 101.9) (width 0.4) (layer "F.Cu") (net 7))
 (segment (start 157.85 101.9) (end 157.85 100.18) (width 0.4) (layer "F.Cu") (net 7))
 (segment (start 158.3 98.76) (end 158.3 98.17701) (width 0.4) (layer "F.Cu") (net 7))
 (segment (start 142.55 101.9) (end 143.25 101.2) (width 0.4) (layer "F.Cu") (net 7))
 (segment (start 157.85 100.18) (end 158.3 99.73) (width 0.4) (layer "F.Cu") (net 7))
 (segment (start 141.05 101.925) (end 140.975 101.85) (width 0.4) (layer "F.Cu") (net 5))
 (segment (start 140.7 103.9) (end 141.05 103.9) (width 0.4) (layer "F.Cu") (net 5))
 (segment (start 141.05 103.9) (end 141.05 101.925) (width 0.4) (layer "F.Cu") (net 5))
 (segment (start 139.85 106.4) (end 140.35 106.9) (width 0.4) (layer "F.Cu") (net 3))
 (segment (start 140.35 106.9) (end 141.05 106.9) (width 0.4) (layer "F.Cu") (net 3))
 (segment (start 139.05 106.4) (end 139.85 106.4) (width 0.4) (layer "F.Cu") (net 3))
 (segment (start 141.05 106.75) (end 141.05 106.9) (width 0.4) (layer "F.Cu") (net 3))
 (segment (start 141.85 108.95) (end 142.55 108.25) (width 0.4) (layer "F.Cu") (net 1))
 (segment (start 142.55 108.25) (end 142.55 106.9) (width 0.4) (layer "F.Cu") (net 1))
 (segment (start 140.975 108.95) (end 141.85 108.95) (width 0.4) (layer "F.Cu") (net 1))
 (segment (start 139 104.35) (end 137.95 105.4) (width 0.4) (layer "F.Cu") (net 4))
 (segment (start 137.95 105.4) (end 136.45 105.4) (width 0.4) (layer "F.Cu") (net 4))
 (segment (start 139.05 104.35) (end 139 104.35) (width 0.4) (layer "F.Cu") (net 4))
 (segment (start 138.925 108.95) (end 138.925 108.925) (width 0.4) (layer "F.Cu") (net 2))
 (segment (start 137.94 107.94) (end 136.45 107.94) (width 0.4) (layer "F.Cu") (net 2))
 (segment (start 138.925 108.925) (end 137.94 107.94) (width 0.4) (layer "F.Cu") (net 2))
 (segment (start 138.925 101.85) (end 138.925 101.925) (width 0.4) (layer "F.Cu") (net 6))
 (segment (start 138.925 101.925) (end 137.99 102.86) (width 0.4) (layer "F.Cu") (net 6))
 (segment (start 137.99 102.86) (end 136.45 102.86) (width 0.4) (layer "F.Cu") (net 6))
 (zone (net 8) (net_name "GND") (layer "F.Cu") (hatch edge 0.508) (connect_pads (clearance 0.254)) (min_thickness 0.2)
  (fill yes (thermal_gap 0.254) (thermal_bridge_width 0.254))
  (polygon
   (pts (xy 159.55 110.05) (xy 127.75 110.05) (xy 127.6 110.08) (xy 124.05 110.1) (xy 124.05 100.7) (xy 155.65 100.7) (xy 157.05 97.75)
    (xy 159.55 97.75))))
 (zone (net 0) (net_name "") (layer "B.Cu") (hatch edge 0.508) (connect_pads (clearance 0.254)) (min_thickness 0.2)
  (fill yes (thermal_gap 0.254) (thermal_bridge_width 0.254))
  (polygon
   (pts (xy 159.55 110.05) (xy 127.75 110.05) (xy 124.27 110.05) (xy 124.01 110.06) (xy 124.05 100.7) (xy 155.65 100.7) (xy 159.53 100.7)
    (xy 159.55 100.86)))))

